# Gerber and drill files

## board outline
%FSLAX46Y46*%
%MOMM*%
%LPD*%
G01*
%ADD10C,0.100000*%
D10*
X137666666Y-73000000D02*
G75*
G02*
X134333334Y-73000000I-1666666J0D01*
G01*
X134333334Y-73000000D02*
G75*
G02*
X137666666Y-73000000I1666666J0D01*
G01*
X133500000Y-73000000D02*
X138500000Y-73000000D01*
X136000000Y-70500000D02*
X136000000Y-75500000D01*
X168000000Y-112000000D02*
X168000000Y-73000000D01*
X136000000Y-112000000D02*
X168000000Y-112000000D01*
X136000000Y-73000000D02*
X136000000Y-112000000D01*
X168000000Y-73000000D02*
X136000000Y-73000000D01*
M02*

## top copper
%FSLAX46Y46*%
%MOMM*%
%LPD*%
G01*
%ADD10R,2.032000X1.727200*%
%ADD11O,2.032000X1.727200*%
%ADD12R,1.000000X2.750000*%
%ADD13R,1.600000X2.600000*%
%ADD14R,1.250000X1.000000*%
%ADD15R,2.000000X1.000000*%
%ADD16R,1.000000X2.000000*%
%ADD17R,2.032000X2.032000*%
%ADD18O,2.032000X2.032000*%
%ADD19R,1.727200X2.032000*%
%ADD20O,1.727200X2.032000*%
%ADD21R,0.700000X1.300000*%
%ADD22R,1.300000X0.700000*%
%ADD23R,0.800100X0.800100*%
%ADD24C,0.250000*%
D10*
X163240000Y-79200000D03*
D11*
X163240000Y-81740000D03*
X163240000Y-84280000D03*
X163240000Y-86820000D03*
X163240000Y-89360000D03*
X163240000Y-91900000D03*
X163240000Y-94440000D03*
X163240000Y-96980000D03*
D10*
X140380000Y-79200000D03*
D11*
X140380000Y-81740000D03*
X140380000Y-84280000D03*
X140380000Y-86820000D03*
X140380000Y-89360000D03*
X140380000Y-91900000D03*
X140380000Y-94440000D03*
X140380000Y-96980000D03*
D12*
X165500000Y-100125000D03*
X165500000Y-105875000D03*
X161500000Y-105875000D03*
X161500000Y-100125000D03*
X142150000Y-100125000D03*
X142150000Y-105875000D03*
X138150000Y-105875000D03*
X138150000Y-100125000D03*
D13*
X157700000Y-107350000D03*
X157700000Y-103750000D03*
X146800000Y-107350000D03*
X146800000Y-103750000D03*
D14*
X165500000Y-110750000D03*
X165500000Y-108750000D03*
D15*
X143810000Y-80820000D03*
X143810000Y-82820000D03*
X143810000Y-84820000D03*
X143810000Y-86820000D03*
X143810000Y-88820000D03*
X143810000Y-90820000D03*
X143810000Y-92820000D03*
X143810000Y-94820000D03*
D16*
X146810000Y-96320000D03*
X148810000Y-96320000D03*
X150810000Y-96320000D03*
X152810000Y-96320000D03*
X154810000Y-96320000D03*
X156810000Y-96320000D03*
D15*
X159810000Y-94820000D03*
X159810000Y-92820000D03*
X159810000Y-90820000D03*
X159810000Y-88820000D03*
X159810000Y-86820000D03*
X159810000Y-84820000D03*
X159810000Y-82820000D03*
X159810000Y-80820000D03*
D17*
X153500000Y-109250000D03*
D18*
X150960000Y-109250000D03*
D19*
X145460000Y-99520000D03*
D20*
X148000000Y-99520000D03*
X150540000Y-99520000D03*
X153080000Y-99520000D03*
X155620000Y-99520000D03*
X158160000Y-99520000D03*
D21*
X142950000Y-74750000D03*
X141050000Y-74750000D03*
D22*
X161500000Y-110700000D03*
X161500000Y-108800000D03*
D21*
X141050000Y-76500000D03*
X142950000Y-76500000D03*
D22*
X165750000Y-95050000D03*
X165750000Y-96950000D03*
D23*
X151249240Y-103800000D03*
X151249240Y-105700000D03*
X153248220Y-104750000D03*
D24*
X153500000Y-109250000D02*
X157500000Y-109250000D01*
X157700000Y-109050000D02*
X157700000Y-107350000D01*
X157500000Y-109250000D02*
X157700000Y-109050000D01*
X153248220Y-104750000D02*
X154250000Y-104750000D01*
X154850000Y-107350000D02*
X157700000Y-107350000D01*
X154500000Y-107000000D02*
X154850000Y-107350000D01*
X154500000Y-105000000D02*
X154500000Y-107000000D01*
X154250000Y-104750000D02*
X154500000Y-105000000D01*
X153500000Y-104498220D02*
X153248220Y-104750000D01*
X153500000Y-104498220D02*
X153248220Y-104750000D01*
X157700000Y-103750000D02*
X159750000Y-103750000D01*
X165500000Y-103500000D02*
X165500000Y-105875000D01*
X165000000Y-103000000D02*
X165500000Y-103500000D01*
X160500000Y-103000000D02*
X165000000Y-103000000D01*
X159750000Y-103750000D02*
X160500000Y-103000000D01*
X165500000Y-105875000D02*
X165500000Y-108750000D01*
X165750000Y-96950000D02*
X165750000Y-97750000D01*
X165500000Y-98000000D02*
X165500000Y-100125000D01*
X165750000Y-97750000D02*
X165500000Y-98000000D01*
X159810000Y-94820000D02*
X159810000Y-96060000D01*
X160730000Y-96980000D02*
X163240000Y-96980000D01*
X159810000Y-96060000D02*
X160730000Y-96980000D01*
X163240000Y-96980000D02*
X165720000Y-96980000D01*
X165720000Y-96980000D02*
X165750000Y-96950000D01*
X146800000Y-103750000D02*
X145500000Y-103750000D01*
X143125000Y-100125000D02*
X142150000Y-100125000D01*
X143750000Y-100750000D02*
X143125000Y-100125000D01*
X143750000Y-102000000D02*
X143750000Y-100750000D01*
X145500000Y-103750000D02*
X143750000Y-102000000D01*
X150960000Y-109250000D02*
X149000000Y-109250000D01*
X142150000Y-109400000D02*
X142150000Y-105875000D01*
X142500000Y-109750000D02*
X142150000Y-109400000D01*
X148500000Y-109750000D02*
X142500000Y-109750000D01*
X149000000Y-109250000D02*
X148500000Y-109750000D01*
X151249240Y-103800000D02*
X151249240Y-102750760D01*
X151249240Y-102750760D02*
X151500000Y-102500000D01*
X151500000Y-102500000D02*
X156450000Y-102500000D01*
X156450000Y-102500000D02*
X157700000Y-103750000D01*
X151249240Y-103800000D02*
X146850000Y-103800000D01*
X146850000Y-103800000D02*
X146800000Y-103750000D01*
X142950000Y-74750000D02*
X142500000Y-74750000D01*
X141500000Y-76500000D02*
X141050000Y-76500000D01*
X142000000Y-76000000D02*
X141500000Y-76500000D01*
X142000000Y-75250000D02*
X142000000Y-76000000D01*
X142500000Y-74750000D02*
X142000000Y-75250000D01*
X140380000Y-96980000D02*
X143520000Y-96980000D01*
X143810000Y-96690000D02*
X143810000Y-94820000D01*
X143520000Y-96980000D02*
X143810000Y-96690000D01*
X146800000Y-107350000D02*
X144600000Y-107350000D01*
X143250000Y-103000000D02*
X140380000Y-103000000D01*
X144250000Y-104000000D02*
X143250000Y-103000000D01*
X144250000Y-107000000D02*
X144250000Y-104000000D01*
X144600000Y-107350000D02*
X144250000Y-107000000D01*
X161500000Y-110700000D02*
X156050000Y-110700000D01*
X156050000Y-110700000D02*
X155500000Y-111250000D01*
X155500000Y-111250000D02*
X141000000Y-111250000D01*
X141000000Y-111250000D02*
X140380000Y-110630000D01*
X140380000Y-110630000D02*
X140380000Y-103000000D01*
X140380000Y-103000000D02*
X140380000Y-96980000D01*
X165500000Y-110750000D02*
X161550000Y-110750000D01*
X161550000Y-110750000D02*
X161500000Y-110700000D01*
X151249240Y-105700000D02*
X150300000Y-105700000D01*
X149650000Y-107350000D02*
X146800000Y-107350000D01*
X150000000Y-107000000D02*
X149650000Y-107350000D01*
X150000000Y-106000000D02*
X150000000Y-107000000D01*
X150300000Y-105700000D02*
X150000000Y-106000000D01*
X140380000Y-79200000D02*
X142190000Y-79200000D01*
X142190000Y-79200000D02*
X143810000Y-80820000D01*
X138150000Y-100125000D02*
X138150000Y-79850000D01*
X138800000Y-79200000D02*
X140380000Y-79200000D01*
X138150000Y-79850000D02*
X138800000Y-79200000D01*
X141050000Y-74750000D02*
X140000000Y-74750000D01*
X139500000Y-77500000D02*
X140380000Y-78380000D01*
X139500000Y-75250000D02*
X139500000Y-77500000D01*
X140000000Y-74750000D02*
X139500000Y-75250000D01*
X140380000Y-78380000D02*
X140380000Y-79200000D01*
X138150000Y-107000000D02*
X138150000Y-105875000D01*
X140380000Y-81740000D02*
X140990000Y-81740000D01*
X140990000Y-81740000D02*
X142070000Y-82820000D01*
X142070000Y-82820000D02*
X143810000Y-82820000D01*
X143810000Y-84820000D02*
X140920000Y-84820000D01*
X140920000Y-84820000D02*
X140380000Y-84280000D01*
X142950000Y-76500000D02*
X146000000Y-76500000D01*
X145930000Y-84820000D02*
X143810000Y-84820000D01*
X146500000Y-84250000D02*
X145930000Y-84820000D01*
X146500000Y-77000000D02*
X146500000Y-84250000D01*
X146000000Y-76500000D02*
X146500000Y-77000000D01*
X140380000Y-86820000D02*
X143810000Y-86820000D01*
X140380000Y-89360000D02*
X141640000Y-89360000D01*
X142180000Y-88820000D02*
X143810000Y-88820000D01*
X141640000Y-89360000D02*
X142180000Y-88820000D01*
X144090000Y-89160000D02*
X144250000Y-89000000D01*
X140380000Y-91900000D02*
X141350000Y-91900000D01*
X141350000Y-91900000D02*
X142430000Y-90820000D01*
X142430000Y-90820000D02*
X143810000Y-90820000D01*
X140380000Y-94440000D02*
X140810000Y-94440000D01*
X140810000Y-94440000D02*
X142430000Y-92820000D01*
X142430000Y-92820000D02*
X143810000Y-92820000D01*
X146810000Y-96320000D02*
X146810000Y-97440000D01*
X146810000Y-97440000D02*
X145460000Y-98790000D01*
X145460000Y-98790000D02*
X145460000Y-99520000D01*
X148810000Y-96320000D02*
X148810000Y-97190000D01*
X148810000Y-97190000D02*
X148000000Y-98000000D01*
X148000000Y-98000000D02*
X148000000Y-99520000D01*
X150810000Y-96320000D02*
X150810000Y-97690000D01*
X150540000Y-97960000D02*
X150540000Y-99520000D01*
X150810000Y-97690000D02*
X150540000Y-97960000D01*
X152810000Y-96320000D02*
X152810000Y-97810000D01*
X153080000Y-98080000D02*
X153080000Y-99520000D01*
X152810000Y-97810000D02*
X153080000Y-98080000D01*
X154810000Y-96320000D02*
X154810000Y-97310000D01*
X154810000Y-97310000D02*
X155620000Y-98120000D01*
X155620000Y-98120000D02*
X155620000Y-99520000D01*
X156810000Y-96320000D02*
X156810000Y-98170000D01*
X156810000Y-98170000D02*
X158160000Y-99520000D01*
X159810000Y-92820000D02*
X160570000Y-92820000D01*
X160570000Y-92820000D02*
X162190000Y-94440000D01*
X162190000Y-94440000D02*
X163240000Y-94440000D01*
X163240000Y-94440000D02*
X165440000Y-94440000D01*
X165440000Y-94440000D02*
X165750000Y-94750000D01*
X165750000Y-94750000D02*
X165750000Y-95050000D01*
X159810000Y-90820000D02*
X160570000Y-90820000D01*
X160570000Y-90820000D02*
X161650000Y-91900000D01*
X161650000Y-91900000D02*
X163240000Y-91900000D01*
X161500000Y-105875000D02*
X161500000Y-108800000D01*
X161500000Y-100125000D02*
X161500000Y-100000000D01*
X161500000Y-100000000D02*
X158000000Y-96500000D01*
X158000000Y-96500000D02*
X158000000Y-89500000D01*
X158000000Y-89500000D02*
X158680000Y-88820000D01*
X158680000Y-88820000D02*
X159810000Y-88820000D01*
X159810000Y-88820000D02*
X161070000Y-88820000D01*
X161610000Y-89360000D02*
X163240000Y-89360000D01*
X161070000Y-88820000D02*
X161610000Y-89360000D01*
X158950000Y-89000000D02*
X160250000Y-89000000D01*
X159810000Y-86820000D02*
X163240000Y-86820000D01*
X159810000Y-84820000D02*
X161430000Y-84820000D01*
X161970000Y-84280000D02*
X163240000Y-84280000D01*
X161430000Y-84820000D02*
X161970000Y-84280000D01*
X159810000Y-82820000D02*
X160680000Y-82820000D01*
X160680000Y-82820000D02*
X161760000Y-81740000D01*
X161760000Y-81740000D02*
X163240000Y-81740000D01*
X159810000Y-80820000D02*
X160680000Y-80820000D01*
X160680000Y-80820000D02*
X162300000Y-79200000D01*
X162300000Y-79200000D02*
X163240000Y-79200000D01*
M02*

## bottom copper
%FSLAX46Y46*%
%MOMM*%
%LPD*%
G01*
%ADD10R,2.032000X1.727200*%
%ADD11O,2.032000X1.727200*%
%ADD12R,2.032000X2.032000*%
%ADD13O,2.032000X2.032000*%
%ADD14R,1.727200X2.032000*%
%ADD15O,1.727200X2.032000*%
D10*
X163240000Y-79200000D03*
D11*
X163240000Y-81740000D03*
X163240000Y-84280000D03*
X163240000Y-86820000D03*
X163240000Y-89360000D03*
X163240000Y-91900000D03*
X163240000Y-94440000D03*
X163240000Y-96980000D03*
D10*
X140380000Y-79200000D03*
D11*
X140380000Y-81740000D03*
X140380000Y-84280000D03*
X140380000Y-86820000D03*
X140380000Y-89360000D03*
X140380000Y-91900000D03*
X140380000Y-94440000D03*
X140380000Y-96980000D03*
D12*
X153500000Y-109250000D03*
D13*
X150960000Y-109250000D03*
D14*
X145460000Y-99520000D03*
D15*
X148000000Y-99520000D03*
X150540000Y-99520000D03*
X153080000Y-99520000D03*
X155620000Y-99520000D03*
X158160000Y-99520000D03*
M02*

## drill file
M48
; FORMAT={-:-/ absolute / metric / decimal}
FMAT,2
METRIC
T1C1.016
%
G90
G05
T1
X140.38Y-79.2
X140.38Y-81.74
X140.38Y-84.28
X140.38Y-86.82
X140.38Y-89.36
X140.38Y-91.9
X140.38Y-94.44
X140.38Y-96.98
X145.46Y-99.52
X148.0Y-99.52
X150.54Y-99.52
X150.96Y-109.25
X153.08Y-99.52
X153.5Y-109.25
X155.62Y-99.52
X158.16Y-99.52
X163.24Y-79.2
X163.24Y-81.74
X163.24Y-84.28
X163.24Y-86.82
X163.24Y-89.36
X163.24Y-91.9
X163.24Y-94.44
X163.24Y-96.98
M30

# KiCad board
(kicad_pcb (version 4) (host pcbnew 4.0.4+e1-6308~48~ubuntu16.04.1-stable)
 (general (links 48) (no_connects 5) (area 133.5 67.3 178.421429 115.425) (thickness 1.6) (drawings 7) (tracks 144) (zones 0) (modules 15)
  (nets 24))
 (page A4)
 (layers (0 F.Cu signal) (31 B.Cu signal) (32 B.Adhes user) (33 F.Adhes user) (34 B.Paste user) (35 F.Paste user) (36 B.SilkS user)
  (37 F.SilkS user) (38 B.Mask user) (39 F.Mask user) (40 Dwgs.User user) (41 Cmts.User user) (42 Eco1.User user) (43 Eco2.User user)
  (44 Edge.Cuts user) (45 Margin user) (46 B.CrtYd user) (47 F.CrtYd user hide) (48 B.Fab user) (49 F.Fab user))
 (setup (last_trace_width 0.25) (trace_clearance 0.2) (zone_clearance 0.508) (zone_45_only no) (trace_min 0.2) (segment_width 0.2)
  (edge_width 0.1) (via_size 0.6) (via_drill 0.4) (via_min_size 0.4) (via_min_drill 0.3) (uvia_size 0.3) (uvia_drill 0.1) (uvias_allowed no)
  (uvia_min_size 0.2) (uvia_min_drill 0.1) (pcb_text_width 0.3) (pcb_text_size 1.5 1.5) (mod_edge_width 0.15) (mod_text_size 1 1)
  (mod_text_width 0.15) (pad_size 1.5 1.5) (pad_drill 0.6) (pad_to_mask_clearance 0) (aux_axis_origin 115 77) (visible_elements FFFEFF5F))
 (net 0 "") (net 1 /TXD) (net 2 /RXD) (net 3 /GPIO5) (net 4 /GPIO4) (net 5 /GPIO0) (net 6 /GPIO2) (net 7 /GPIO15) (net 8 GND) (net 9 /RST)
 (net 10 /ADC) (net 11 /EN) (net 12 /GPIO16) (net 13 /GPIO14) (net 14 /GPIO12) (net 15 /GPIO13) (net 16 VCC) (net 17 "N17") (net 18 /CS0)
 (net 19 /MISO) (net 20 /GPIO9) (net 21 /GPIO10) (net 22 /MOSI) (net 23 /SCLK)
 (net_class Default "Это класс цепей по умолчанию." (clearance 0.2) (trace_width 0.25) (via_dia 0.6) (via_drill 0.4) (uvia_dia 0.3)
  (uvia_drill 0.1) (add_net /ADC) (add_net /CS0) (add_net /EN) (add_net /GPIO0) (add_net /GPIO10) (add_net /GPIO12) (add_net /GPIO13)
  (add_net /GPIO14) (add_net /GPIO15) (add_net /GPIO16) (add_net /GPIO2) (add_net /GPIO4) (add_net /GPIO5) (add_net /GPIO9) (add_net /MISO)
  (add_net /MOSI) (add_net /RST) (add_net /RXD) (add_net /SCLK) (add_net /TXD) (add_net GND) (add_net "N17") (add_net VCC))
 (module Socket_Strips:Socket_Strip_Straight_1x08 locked (layer F.Cu) (at 163.24 79.2 270)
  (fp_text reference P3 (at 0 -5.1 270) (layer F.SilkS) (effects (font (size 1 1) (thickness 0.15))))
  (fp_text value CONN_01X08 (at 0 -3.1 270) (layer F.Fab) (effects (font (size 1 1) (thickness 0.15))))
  (pad 1 thru_hole rect (at 0 0 270) (size 1.7272 2.032) (drill 1.016) (layers *.Cu *.Mask F.SilkS) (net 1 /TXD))
  (pad 2 thru_hole oval (at 2.54 0 270) (size 1.7272 2.032) (drill 1.016) (layers *.Cu *.Mask F.SilkS) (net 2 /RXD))
  (pad 3 thru_hole oval (at 5.08 0 270) (size 1.7272 2.032) (drill 1.016) (layers *.Cu *.Mask F.SilkS) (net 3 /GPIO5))
  (pad 4 thru_hole oval (at 7.62 0 270) (size 1.7272 2.032) (drill 1.016) (layers *.Cu *.Mask F.SilkS) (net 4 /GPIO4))
  (pad 5 thru_hole oval (at 10.16 0 270) (size 1.7272 2.032) (drill 1.016) (layers *.Cu *.Mask F.SilkS) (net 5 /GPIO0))
  (pad 6 thru_hole oval (at 12.7 0 270) (size 1.7272 2.032) (drill 1.016) (layers *.Cu *.Mask F.SilkS) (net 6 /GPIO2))
  (pad 7 thru_hole oval (at 15.24 0 270) (size 1.7272 2.032) (drill 1.016) (layers *.Cu *.Mask F.SilkS) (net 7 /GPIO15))
  (pad 8 thru_hole oval (at 17.78 0 270) (size 1.7272 2.032) (drill 1.016) (layers *.Cu *.Mask F.SilkS) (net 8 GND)))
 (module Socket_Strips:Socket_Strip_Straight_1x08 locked (layer F.Cu) (at 140.38 79.2 270)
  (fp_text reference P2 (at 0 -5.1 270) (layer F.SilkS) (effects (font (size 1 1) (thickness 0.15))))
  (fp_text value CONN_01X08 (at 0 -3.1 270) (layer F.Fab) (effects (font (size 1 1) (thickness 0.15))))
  (pad 1 thru_hole rect (at 0 0 270) (size 1.7272 2.032) (drill 1.016) (layers *.Cu *.Mask F.SilkS) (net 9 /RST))
  (pad 2 thru_hole oval (at 2.54 0 270) (size 1.7272 2.032) (drill 1.016) (layers *.Cu *.Mask F.SilkS) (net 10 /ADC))
  (pad 3 thru_hole oval (at 5.08 0 270) (size 1.7272 2.032) (drill 1.016) (layers *.Cu *.Mask F.SilkS) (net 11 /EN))
  (pad 4 thru_hole oval (at 7.62 0 270) (size 1.7272 2.032) (drill 1.016) (layers *.Cu *.Mask F.SilkS) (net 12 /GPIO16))
  (pad 5 thru_hole oval (at 10.16 0 270) (size 1.7272 2.032) (drill 1.016) (layers *.Cu *.Mask F.SilkS) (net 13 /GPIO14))
  (pad 6 thru_hole oval (at 12.7 0 270) (size 1.7272 2.032) (drill 1.016) (layers *.Cu *.Mask F.SilkS) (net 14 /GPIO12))
  (pad 7 thru_hole oval (at 15.24 0 270) (size 1.7272 2.032) (drill 1.016) (layers *.Cu *.Mask F.SilkS) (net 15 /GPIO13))
  (pad 8 thru_hole oval (at 17.78 0 270) (size 1.7272 2.032) (drill 1.016) (layers *.Cu *.Mask F.SilkS) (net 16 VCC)))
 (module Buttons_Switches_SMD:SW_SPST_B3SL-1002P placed (layer F.Cu) (at 163.5 103 270)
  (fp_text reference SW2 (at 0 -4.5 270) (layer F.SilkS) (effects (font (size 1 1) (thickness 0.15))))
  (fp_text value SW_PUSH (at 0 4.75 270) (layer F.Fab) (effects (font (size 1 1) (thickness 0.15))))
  (pad 1 smd rect (at -2.875 -2 270) (size 2.75 1) (layers F.Cu F.Paste F.Mask) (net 8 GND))
  (pad 1 smd rect (at 2.875 -2 270) (size 2.75 1) (layers F.Cu F.Paste F.Mask) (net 8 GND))
  (pad 2 smd rect (at 2.875 2 270) (size 2.75 1) (layers F.Cu F.Paste F.Mask) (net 5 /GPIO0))
  (pad 2 smd rect (at -2.875 2 270) (size 2.75 1) (layers F.Cu F.Paste F.Mask) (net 5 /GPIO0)))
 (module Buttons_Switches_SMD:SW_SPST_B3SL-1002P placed (layer F.Cu) (at 140.15 103 270)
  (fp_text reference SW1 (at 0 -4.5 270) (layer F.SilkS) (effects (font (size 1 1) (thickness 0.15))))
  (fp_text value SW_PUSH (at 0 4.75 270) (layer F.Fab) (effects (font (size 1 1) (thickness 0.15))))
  (pad 1 smd rect (at -2.875 -2 270) (size 2.75 1) (layers F.Cu F.Paste F.Mask) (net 8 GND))
  (pad 1 smd rect (at 2.875 -2 270) (size 2.75 1) (layers F.Cu F.Paste F.Mask) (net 8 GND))
  (pad 2 smd rect (at 2.875 2 270) (size 2.75 1) (layers F.Cu F.Paste F.Mask) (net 9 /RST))
  (pad 2 smd rect (at -2.875 2 270) (size 2.75 1) (layers F.Cu F.Paste F.Mask) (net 9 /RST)))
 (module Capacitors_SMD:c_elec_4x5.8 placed (layer F.Cu) (at 157.7 105.55 90)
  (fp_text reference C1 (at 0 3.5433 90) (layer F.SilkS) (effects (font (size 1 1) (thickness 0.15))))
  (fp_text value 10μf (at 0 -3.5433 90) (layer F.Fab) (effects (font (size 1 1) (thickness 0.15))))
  (pad 1 smd rect (at -1.8 0 270) (size 2.6 1.6) (layers F.Cu F.Paste F.Mask) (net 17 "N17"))
  (pad 2 smd rect (at 1.8 0 270) (size 2.6 1.6) (layers F.Cu F.Paste F.Mask) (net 8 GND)))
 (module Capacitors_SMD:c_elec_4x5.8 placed (layer F.Cu) (at 146.8 105.55 90)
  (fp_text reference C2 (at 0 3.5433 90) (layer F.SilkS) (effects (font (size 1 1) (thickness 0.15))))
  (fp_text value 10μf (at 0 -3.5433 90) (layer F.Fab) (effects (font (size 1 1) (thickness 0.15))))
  (pad 1 smd rect (at -1.8 0 270) (size 2.6 1.6) (layers F.Cu F.Paste F.Mask) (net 16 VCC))
  (pad 2 smd rect (at 1.8 0 270) (size 2.6 1.6) (layers F.Cu F.Paste F.Mask) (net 8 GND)))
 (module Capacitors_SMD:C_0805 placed (layer F.Cu) (at 165.5 109.75 90)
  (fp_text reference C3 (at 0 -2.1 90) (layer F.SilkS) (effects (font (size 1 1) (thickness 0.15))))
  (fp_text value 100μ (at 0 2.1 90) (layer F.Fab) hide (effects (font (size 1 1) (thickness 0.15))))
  (pad 1 smd rect (at -1 0 90) (size 1 1.25) (layers F.Cu F.Paste F.Mask) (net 16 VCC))
  (pad 2 smd rect (at 1 0 90) (size 1 1.25) (layers F.Cu F.Paste F.Mask) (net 8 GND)))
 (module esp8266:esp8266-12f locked (layer F.Cu) (at 151.81 86.82)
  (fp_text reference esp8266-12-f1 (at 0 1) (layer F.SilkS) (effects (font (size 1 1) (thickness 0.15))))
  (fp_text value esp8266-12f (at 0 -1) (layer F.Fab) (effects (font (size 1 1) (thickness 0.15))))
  (pad 1 smd rect (at -8 -6) (size 2 1) (layers F.Cu F.Paste F.Mask) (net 9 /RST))
  (pad 2 smd rect (at -8 -4) (size 2 1) (layers F.Cu F.Paste F.Mask) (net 10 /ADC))
  (pad 3 smd rect (at -8 -2) (size 2 1) (layers F.Cu F.Paste F.Mask) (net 11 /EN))
  (pad 4 smd rect (at -8 0) (size 2 1) (layers F.Cu F.Paste F.Mask) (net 12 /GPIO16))
  (pad 5 smd rect (at -8 2) (size 2 1) (layers F.Cu F.Paste F.Mask) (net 13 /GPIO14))
  (pad 6 smd rect (at -8 4) (size 2 1) (layers F.Cu F.Paste F.Mask) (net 14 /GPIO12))
  (pad 7 smd rect (at -8 6) (size 2 1) (layers F.Cu F.Paste F.Mask) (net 15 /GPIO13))
  (pad 8 smd rect (at -8 8) (size 2 1) (layers F.Cu F.Paste F.Mask) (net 16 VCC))
  (pad 9 smd rect (at -5 9.5) (size 1 2) (layers F.Cu F.Paste F.Mask) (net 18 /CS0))
  (pad 10 smd rect (at -3 9.5) (size 1 2) (layers F.Cu F.Paste F.Mask) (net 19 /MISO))
  (pad 11 smd rect (at -1 9.5) (size 1 2) (layers F.Cu F.Paste F.Mask) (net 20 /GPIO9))
  (pad 12 smd rect (at 1 9.5) (size 1 2) (layers F.Cu F.Paste F.Mask) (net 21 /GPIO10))
  (pad 13 smd rect (at 3 9.5) (size 1 2) (layers F.Cu F.Paste F.Mask) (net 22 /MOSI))
  (pad 14 smd rect (at 5 9.5) (size 1 2) (layers F.Cu F.Paste F.Mask) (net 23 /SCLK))
  (pad 15 smd rect (at 8 8) (size 2 1) (layers F.Cu F.Paste F.Mask) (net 8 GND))
  (pad 16 smd rect (at 8 6) (size 2 1) (layers F.Cu F.Paste F.Mask) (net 7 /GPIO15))
  (pad 17 smd rect (at 8 4) (size 2 1) (layers F.Cu F.Paste F.Mask) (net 6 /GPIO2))
  (pad 18 smd rect (at 8 2) (size 2 1) (layers F.Cu F.Paste F.Mask) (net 5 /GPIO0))
  (pad 19 smd rect (at 8 0) (size 2 1) (layers F.Cu F.Paste F.Mask) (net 4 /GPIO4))
  (pad 20 smd rect (at 8 -2) (size 2 1) (layers F.Cu F.Paste F.Mask) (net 3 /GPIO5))
  (pad 21 smd rect (at 8 -4) (size 2 1) (layers F.Cu F.Paste F.Mask) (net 2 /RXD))
  (pad 22 smd rect (at 8 -6) (size 2 1) (layers F.Cu F.Paste F.Mask) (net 1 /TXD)))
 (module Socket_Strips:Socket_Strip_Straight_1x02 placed (layer F.Cu) (at 153.5 109.25 180)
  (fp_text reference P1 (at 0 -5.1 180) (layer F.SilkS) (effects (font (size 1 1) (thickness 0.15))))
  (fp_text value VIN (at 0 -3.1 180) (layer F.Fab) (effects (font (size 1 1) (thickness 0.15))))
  (pad 1 thru_hole rect (at 0 0 180) (size 2.032 2.032) (drill 1.016) (layers *.Cu *.Mask F.SilkS) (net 17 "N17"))
  (pad 2 thru_hole oval (at 2.54 0 180) (size 2.032 2.032) (drill 1.016) (layers *.Cu *.Mask F.SilkS) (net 8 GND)))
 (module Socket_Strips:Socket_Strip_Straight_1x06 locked (layer F.Cu) (at 145.46 99.52)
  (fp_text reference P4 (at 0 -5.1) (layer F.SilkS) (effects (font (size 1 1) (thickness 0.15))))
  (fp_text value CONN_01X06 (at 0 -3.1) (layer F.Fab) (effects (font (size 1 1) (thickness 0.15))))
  (pad 1 thru_hole rect (at 0 0) (size 1.7272 2.032) (drill 1.016) (layers *.Cu *.Mask F.SilkS) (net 18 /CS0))
  (pad 2 thru_hole oval (at 2.54 0) (size 1.7272 2.032) (drill 1.016) (layers *.Cu *.Mask F.SilkS) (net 19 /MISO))
  (pad 3 thru_hole oval (at 5.08 0) (size 1.7272 2.032) (drill 1.016) (layers *.Cu *.Mask F.SilkS) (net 20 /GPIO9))
  (pad 4 thru_hole oval (at 7.62 0) (size 1.7272 2.032) (drill 1.016) (layers *.Cu *.Mask F.SilkS) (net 21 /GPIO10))
  (pad 5 thru_hole oval (at 10.16 0) (size 1.7272 2.032) (drill 1.016) (layers *.Cu *.Mask F.SilkS) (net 22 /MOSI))
  (pad 6 thru_hole oval (at 12.7 0) (size 1.7272 2.032) (drill 1.016) (layers *.Cu *.Mask F.SilkS) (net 23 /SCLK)))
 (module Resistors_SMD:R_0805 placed (layer F.Cu) (at 142 74.75 180)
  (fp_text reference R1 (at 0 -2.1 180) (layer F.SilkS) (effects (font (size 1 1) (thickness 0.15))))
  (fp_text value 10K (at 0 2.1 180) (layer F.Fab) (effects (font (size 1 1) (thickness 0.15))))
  (pad 1 smd rect (at -0.95 0 180) (size 0.7 1.3) (layers F.Cu F.Paste F.Mask) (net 16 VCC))
  (pad 2 smd rect (at 0.95 0 180) (size 0.7 1.3) (layers F.Cu F.Paste F.Mask) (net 9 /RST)))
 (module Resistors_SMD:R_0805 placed (layer F.Cu) (at 161.5 109.75 90)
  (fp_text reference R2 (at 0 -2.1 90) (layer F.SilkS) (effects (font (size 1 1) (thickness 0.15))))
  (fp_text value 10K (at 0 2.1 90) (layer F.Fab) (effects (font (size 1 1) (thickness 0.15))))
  (pad 1 smd rect (at -0.95 0 90) (size 0.7 1.3) (layers F.Cu F.Paste F.Mask) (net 16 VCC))
  (pad 2 smd rect (at 0.95 0 90) (size 0.7 1.3) (layers F.Cu F.Paste F.Mask) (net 5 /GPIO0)))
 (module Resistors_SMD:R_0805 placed (layer F.Cu) (at 142 76.5)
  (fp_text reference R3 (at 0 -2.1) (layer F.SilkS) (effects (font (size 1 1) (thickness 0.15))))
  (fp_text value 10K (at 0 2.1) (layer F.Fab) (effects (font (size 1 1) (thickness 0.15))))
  (pad 1 smd rect (at -0.95 0) (size 0.7 1.3) (layers F.Cu F.Paste F.Mask) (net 16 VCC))
  (pad 2 smd rect (at 0.95 0) (size 0.7 1.3) (layers F.Cu F.Paste F.Mask) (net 11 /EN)))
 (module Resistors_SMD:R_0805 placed (layer F.Cu) (at 165.75 96 270)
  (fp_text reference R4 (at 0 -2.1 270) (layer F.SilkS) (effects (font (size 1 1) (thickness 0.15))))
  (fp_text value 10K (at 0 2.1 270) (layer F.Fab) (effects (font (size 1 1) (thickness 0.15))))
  (pad 1 smd rect (at -0.95 0 270) (size 0.7 1.3) (layers F.Cu F.Paste F.Mask) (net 7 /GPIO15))
  (pad 2 smd rect (at 0.95 0 270) (size 0.7 1.3) (layers F.Cu F.Paste F.Mask) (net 8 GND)))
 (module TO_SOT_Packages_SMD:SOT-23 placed (layer F.Cu) (at 152.25 104.75 270)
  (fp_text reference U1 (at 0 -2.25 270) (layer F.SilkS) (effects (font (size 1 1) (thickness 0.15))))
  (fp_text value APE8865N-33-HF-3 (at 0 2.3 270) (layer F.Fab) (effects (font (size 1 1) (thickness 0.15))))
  (pad 1 smd rect (at -0.95 1.00076 270) (size 0.8001 0.8001) (layers F.Cu F.Paste F.Mask) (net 8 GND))
  (pad 2 smd rect (at 0.95 1.00076 270) (size 0.8001 0.8001) (layers F.Cu F.Paste F.Mask) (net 16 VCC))
  (pad 3 smd rect (at 0 -0.99822 270) (size 0.8001 0.8001) (layers F.Cu F.Paste F.Mask) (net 17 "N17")))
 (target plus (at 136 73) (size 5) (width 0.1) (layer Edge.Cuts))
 (gr_line (start 168 112) (end 168 73) (angle 90) (layer Edge.Cuts) (width 0.1))
 (gr_line (start 136 112) (end 168 112) (angle 90) (layer Edge.Cuts) (width 0.1))
 (gr_line (start 136 73) (end 136 112) (angle 90) (layer Edge.Cuts) (width 0.1))
 (gr_line (start 168 73) (end 136 73) (angle 90) (layer Edge.Cuts) (width 0.1))
 (segment (start 153.5 109.25) (end 157.5 109.25) (width 0.25) (layer F.Cu) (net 17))
 (segment (start 157.7 109.05) (end 157.7 107.35) (width 0.25) (layer F.Cu) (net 17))
 (segment (start 157.5 109.25) (end 157.7 109.05) (width 0.25) (layer F.Cu) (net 17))
 (segment (start 153.24822 104.75) (end 154.25 104.75) (width 0.25) (layer F.Cu) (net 17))
 (segment (start 154.85 107.35) (end 157.7 107.35) (width 0.25) (layer F.Cu) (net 17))
 (segment (start 154.5 107) (end 154.85 107.35) (width 0.25) (layer F.Cu) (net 17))
 (segment (start 154.5 105) (end 154.5 107) (width 0.25) (layer F.Cu) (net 17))
 (segment (start 154.25 104.75) (end 154.5 105) (width 0.25) (layer F.Cu) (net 17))
 (segment (start 153.5 104.49822) (end 153.24822 104.75) (width 0.25) (layer F.Cu) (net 17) (status 30))
 (segment (start 153.5 104.49822) (end 153.24822 104.75) (width 0.25) (layer F.Cu) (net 17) (status 30))
 (segment (start 157.7 103.75) (end 159.75 103.75) (width 0.25) (layer F.Cu) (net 8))
 (segment (start 165.5 103.5) (end 165.5 105.875) (width 0.25) (layer F.Cu) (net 8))
 (segment (start 165 103) (end 165.5 103.5) (width 0.25) (layer F.Cu) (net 8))
 (segment (start 160.5 103) (end 165 103) (width 0.25) (layer F.Cu) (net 8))
 (segment (start 159.75 103.75) (end 160.5 103) (width 0.25) (layer F.Cu) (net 8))
 (segment (start 165.5 105.875) (end 165.5 108.75) (width 0.25) (layer F.Cu) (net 8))
 (segment (start 165.75 96.95) (end 165.75 97.75) (width 0.25) (layer F.Cu) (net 8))
 (segment (start 165.5 98) (end 165.5 100.125) (width 0.25) (layer F.Cu) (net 8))
 (segment (start 165.75 97.75) (end 165.5 98) (width 0.25) (layer F.Cu) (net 8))
 (segment (start 159.81 94.82) (end 159.81 96.06) (width 0.25) (layer F.Cu) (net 8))
 (segment (start 160.73 96.98) (end 163.24 96.98) (width 0.25) (layer F.Cu) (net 8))
 (segment (start 159.81 96.06) (end 160.73 96.98) (width 0.25) (layer F.Cu) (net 8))
 (segment (start 163.24 96.98) (end 165.72 96.98) (width 0.25) (layer F.Cu) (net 8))
 (segment (start 165.72 96.98) (end 165.75 96.95) (width 0.25) (layer F.Cu) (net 8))
 (segment (start 146.8 103.75) (end 145.5 103.75) (width 0.25) (layer F.Cu) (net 8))
 (segment (start 143.125 100.125) (end 142.15 100.125) (width 0.25) (layer F.Cu) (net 8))
 (segment (start 143.75 100.75) (end 143.125 100.125) (width 0.25) (layer F.Cu) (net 8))
 (segment (start 143.75 102) (end 143.75 100.75) (width 0.25) (layer F.Cu) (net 8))
 (segment (start 145.5 103.75) (end 143.75 102) (width 0.25) (layer F.Cu) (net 8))
 (segment (start 150.96 109.25) (end 149 109.25) (width 0.25) (layer F.Cu) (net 8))
 (segment (start 142.15 109.4) (end 142.15 105.875) (width 0.25) (layer F.Cu) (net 8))
 (segment (start 142.5 109.75) (end 142.15 109.4) (width 0.25) (layer F.Cu) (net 8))
 (segment (start 148.5 109.75) (end 142.5 109.75) (width 0.25) (layer F.Cu) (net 8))
 (segment (start 149 109.25) (end 148.5 109.75) (width 0.25) (layer F.Cu) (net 8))
 (segment (start 151.24924 103.8) (end 151.24924 102.75076) (width 0.25) (layer F.Cu) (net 8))
 (segment (start 151.24924 102.75076) (end 151.5 102.5) (width 0.25) (layer F.Cu) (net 8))
 (segment (start 151.5 102.5) (end 156.45 102.5) (width 0.25) (layer F.Cu) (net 8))
 (segment (start 156.45 102.5) (end 157.7 103.75) (width 0.25) (layer F.Cu) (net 8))
 (segment (start 151.24924 103.8) (end 146.85 103.8) (width 0.25) (layer F.Cu) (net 8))
 (segment (start 146.85 103.8) (end 146.8 103.75) (width 0.25) (layer F.Cu) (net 8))
 (segment (start 142.95 74.75) (end 142.5 74.75) (width 0.25) (layer F.Cu) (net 16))
 (segment (start 141.5 76.5) (end 141.05 76.5) (width 0.25) (layer F.Cu) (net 16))
 (segment (start 142 76) (end 141.5 76.5) (width 0.25) (layer F.Cu) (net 16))
 (segment (start 142 75.25) (end 142 76) (width 0.25) (layer F.Cu) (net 16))
 (segment (start 142.5 74.75) (end 142 75.25) (width 0.25) (layer F.Cu) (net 16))
 (segment (start 140.38 96.98) (end 143.52 96.98) (width 0.25) (layer F.Cu) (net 16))
 (segment (start 143.81 96.69) (end 143.81 94.82) (width 0.25) (layer F.Cu) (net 16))
 (segment (start 143.52 96.98) (end 143.81 96.69) (width 0.25) (layer F.Cu) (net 16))
 (segment (start 146.8 107.35) (end 144.6 107.35) (width 0.25) (layer F.Cu) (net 16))
 (segment (start 143.25 103) (end 140.38 103) (width 0.25) (layer F.Cu) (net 16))
 (segment (start 144.25 104) (end 143.25 103) (width 0.25) (layer F.Cu) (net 16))
 (segment (start 144.25 107) (end 144.25 104) (width 0.25) (layer F.Cu) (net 16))
 (segment (start 144.6 107.35) (end 144.25 107) (width 0.25) (layer F.Cu) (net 16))
 (segment (start 161.5 110.7) (end 156.05 110.7) (width 0.25) (layer F.Cu) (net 16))
 (segment (start 156.05 110.7) (end 155.5 111.25) (width 0.25) (layer F.Cu) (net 16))
 (segment (start 155.5 111.25) (end 141 111.25) (width 0.25) (layer F.Cu) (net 16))
 (segment (start 141 111.25) (end 140.38 110.63) (width 0.25) (layer F.Cu) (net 16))
 (segment (start 140.38 110.63) (end 140.38 103) (width 0.25) (layer F.Cu) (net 16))
 (segment (start 140.38 103) (end 140.38 96.98) (width 0.25) (layer F.Cu) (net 16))
 (segment (start 165.5 110.75) (end 161.55 110.75) (width 0.25) (layer F.Cu) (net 16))
 (segment (start 161.55 110.75) (end 161.5 110.7) (width 0.25) (layer F.Cu) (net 16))
 (segment (start 151.24924 105.7) (end 150.3 105.7) (width 0.25) (layer F.Cu) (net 16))
 (segment (start 149.65 107.35) (end 146.8 107.35) (width 0.25) (layer F.Cu) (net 16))
 (segment (start 150 107) (end 149.65 107.35) (width 0.25) (layer F.Cu) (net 16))
 (segment (start 150 106) (end 150 107) (width 0.25) (layer F.Cu) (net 16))
 (segment (start 150.3 105.7) (end 150 106) (width 0.25) (layer F.Cu) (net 16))
 (segment (start 140.38 79.2) (end 142.19 79.2) (width 0.25) (layer F.Cu) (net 9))
 (segment (start 142.19 79.2) (end 143.81 80.82) (width 0.25) (layer F.Cu) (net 9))
 (segment (start 138.15 100.125) (end 138.15 79.85) (width 0.25) (layer F.Cu) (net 9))
 (segment (start 138.8 79.2) (end 140.38 79.2) (width 0.25) (layer F.Cu) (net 9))
 (segment (start 138.15 79.85) (end 138.8 79.2) (width 0.25) (layer F.Cu) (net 9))
 (segment (start 141.05 74.75) (end 140 74.75) (width 0.25) (layer F.Cu) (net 9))
 (segment (start 139.5 77.5) (end 140.38 78.38) (width 0.25) (layer F.Cu) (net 9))
 (segment (start 139.5 75.25) (end 139.5 77.5) (width 0.25) (layer F.Cu) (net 9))
 (segment (start 140 74.75) (end 139.5 75.25) (width 0.25) (layer F.Cu) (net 9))
 (segment (start 140.38 78.38) (end 140.38 79.2) (width 0.25) (layer F.Cu) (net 9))
 (segment (start 138.15 107) (end 138.15 105.875) (width 0.25) (layer F.Cu) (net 9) (status 30))
 (segment (start 140.38 81.74) (end 140.99 81.74) (width 0.25) (layer F.Cu) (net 10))
 (segment (start 140.99 81.74) (end 142.07 82.82) (width 0.25) (layer F.Cu) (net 10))
 (segment (start 142.07 82.82) (end 143.81 82.82) (width 0.25) (layer F.Cu) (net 10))
 (segment (start 143.81 84.82) (end 140.92 84.82) (width 0.25) (layer F.Cu) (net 11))
 (segment (start 140.92 84.82) (end 140.38 84.28) (width 0.25) (layer F.Cu) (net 11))
 (segment (start 142.95 76.5) (end 146 76.5) (width 0.25) (layer F.Cu) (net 11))
 (segment (start 145.93 84.82) (end 143.81 84.82) (width 0.25) (layer F.Cu) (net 11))
 (segment (start 146.5 84.25) (end 145.93 84.82) (width 0.25) (layer F.Cu) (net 11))
 (segment (start 146.5 77) (end 146.5 84.25) (width 0.25) (layer F.Cu) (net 11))
 (segment (start 146 76.5) (end 146.5 77) (width 0.25) (layer F.Cu) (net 11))
 (segment (start 140.38 86.82) (end 143.81 86.82) (width 0.25) (layer F.Cu) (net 12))
 (segment (start 140.38 89.36) (end 141.64 89.36) (width 0.25) (layer F.Cu) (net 13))
 (segment (start 142.18 88.82) (end 143.81 88.82) (width 0.25) (layer F.Cu) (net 13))
 (segment (start 141.64 89.36) (end 142.18 88.82) (width 0.25) (layer F.Cu) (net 13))
 (segment (start 144.09 89.16) (end 144.25 89) (width 0.25) (layer F.Cu) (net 13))
 (segment (start 140.38 91.9) (end 141.35 91.9) (width 0.25) (layer F.Cu) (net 14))
 (segment (start 141.35 91.9) (end 142.43 90.82) (width 0.25) (layer F.Cu) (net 14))
 (segment (start 142.43 90.82) (end 143.81 90.82) (width 0.25) (layer F.Cu) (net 14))
 (segment (start 140.38 94.44) (end 140.81 94.44) (width 0.25) (layer F.Cu) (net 15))
 (segment (start 140.81 94.44) (end 142.43 92.82) (width 0.25) (layer F.Cu) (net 15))
 (segment (start 142.43 92.82) (end 143.81 92.82) (width 0.25) (layer F.Cu) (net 15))
 (segment (start 146.81 96.32) (end 146.81 97.44) (width 0.25) (layer F.Cu) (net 18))
 (segment (start 146.81 97.44) (end 145.46 98.79) (width 0.25) (layer F.Cu) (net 18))
 (segment (start 145.46 98.79) (end 145.46 99.52) (width 0.25) (layer F.Cu) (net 18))
 (segment (start 148.81 96.32) (end 148.81 97.19) (width 0.25) (layer F.Cu) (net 19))
 (segment (start 148.81 97.19) (end 148 98) (width 0.25) (layer F.Cu) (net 19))
 (segment (start 148 98) (end 148 99.52) (width 0.25) (layer F.Cu) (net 19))
 (segment (start 150.81 96.32) (end 150.81 97.69) (width 0.25) (layer F.Cu) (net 20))
 (segment (start 150.54 97.96) (end 150.54 99.52) (width 0.25) (layer F.Cu) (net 20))
 (segment (start 150.81 97.69) (end 150.54 97.96) (width 0.25) (layer F.Cu) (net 20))
 (segment (start 152.81 96.32) (end 152.81 97.81) (width 0.25) (layer F.Cu) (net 21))
 (segment (start 153.08 98.08) (end 153.08 99.52) (width 0.25) (layer F.Cu) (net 21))
 (segment (start 152.81 97.81) (end 153.08 98.08) (width 0.25) (layer F.Cu) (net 21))
 (segment (start 154.81 96.32) (end 154.81 97.31) (width 0.25) (layer F.Cu) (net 22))
 (segment (start 154.81 97.31) (end 155.62 98.12) (width 0.25) (layer F.Cu) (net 22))
 (segment (start 155.62 98.12) (end 155.62 99.52) (width 0.25) (layer F.Cu) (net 22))
 (segment (start 156.81 96.32) (end 156.81 98.17) (width 0.25) (layer F.Cu) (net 23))
 (segment (start 156.81 98.17) (end 158.16 99.52) (width 0.25) (layer F.Cu) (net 23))
 (segment (start 159.81 92.82) (end 160.57 92.82) (width 0.25) (layer F.Cu) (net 7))
 (segment (start 160.57 92.82) (end 162.19 94.44) (width 0.25) (layer F.Cu) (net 7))
 (segment (start 162.19 94.44) (end 163.24 94.44) (width 0.25) (layer F.Cu) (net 7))
 (segment (start 163.24 94.44) (end 165.44 94.44) (width 0.25) (layer F.Cu) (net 7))
 (segment (start 165.44 94.44) (end 165.75 94.75) (width 0.25) (layer F.Cu) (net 7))
 (segment (start 165.75 94.75) (end 165.75 95.05) (width 0.25) (layer F.Cu) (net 7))
 (segment (start 159.81 90.82) (end 160.57 90.82) (width 0.25) (layer F.Cu) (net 6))
 (segment (start 160.57 90.82) (end 161.65 91.9) (width 0.25) (layer F.Cu) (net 6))
 (segment (start 161.65 91.9) (end 163.24 91.9) (width 0.25) (layer F.Cu) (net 6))
 (segment (start 161.5 105.875) (end 161.5 108.8) (width 0.25) (layer F.Cu) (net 5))
 (segment (start 161.5 100.125) (end 161.5 100) (width 0.25) (layer F.Cu) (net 5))
 (segment (start 161.5 100) (end 158 96.5) (width 0.25) (layer F.Cu) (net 5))
 (segment (start 158 96.5) (end 158 89.5) (width 0.25) (layer F.Cu) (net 5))
 (segment (start 158 89.5) (end 158.68 88.82) (width 0.25) (layer F.Cu) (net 5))
 (segment (start 158.68 88.82) (end 159.81 88.82) (width 0.25) (layer F.Cu) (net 5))
 (segment (start 159.81 88.82) (end 161.07 88.82) (width 0.25) (layer F.Cu) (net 5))
 (segment (start 161.61 89.36) (end 163.24 89.36) (width 0.25) (layer F.Cu) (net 5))
 (segment (start 161.07 88.82) (end 161.61 89.36) (width 0.25) (layer F.Cu) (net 5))
 (segment (start 158.95 89) (end 160.25 89) (width 0.25) (layer F.Cu) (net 5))
 (segment (start 159.81 86.82) (end 163.24 86.82) (width 0.25) (layer F.Cu) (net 4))
 (segment (start 159.81 84.82) (end 161.43 84.82) (width 0.25) (layer F.Cu) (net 3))
 (segment (start 161.97 84.28) (end 163.24 84.28) (width 0.25) (layer F.Cu) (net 3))
 (segment (start 161.43 84.82) (end 161.97 84.28) (width 0.25) (layer F.Cu) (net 3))
 (segment (start 159.81 82.82) (end 160.68 82.82) (width 0.25) (layer F.Cu) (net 2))
 (segment (start 160.68 82.82) (end 161.76 81.74) (width 0.25) (layer F.Cu) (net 2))
 (segment (start 161.76 81.74) (end 163.24 81.74) (width 0.25) (layer F.Cu) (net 2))
 (segment (start 159.81 80.82) (end 160.68 80.82) (width 0.25) (layer F.Cu) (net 1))
 (segment (start 160.68 80.82) (end 162.3 79.2) (width 0.25) (layer F.Cu) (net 1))
 (segment (start 162.3 79.2) (end 163.24 79.2) (width 0.25) (layer F.Cu) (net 1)))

